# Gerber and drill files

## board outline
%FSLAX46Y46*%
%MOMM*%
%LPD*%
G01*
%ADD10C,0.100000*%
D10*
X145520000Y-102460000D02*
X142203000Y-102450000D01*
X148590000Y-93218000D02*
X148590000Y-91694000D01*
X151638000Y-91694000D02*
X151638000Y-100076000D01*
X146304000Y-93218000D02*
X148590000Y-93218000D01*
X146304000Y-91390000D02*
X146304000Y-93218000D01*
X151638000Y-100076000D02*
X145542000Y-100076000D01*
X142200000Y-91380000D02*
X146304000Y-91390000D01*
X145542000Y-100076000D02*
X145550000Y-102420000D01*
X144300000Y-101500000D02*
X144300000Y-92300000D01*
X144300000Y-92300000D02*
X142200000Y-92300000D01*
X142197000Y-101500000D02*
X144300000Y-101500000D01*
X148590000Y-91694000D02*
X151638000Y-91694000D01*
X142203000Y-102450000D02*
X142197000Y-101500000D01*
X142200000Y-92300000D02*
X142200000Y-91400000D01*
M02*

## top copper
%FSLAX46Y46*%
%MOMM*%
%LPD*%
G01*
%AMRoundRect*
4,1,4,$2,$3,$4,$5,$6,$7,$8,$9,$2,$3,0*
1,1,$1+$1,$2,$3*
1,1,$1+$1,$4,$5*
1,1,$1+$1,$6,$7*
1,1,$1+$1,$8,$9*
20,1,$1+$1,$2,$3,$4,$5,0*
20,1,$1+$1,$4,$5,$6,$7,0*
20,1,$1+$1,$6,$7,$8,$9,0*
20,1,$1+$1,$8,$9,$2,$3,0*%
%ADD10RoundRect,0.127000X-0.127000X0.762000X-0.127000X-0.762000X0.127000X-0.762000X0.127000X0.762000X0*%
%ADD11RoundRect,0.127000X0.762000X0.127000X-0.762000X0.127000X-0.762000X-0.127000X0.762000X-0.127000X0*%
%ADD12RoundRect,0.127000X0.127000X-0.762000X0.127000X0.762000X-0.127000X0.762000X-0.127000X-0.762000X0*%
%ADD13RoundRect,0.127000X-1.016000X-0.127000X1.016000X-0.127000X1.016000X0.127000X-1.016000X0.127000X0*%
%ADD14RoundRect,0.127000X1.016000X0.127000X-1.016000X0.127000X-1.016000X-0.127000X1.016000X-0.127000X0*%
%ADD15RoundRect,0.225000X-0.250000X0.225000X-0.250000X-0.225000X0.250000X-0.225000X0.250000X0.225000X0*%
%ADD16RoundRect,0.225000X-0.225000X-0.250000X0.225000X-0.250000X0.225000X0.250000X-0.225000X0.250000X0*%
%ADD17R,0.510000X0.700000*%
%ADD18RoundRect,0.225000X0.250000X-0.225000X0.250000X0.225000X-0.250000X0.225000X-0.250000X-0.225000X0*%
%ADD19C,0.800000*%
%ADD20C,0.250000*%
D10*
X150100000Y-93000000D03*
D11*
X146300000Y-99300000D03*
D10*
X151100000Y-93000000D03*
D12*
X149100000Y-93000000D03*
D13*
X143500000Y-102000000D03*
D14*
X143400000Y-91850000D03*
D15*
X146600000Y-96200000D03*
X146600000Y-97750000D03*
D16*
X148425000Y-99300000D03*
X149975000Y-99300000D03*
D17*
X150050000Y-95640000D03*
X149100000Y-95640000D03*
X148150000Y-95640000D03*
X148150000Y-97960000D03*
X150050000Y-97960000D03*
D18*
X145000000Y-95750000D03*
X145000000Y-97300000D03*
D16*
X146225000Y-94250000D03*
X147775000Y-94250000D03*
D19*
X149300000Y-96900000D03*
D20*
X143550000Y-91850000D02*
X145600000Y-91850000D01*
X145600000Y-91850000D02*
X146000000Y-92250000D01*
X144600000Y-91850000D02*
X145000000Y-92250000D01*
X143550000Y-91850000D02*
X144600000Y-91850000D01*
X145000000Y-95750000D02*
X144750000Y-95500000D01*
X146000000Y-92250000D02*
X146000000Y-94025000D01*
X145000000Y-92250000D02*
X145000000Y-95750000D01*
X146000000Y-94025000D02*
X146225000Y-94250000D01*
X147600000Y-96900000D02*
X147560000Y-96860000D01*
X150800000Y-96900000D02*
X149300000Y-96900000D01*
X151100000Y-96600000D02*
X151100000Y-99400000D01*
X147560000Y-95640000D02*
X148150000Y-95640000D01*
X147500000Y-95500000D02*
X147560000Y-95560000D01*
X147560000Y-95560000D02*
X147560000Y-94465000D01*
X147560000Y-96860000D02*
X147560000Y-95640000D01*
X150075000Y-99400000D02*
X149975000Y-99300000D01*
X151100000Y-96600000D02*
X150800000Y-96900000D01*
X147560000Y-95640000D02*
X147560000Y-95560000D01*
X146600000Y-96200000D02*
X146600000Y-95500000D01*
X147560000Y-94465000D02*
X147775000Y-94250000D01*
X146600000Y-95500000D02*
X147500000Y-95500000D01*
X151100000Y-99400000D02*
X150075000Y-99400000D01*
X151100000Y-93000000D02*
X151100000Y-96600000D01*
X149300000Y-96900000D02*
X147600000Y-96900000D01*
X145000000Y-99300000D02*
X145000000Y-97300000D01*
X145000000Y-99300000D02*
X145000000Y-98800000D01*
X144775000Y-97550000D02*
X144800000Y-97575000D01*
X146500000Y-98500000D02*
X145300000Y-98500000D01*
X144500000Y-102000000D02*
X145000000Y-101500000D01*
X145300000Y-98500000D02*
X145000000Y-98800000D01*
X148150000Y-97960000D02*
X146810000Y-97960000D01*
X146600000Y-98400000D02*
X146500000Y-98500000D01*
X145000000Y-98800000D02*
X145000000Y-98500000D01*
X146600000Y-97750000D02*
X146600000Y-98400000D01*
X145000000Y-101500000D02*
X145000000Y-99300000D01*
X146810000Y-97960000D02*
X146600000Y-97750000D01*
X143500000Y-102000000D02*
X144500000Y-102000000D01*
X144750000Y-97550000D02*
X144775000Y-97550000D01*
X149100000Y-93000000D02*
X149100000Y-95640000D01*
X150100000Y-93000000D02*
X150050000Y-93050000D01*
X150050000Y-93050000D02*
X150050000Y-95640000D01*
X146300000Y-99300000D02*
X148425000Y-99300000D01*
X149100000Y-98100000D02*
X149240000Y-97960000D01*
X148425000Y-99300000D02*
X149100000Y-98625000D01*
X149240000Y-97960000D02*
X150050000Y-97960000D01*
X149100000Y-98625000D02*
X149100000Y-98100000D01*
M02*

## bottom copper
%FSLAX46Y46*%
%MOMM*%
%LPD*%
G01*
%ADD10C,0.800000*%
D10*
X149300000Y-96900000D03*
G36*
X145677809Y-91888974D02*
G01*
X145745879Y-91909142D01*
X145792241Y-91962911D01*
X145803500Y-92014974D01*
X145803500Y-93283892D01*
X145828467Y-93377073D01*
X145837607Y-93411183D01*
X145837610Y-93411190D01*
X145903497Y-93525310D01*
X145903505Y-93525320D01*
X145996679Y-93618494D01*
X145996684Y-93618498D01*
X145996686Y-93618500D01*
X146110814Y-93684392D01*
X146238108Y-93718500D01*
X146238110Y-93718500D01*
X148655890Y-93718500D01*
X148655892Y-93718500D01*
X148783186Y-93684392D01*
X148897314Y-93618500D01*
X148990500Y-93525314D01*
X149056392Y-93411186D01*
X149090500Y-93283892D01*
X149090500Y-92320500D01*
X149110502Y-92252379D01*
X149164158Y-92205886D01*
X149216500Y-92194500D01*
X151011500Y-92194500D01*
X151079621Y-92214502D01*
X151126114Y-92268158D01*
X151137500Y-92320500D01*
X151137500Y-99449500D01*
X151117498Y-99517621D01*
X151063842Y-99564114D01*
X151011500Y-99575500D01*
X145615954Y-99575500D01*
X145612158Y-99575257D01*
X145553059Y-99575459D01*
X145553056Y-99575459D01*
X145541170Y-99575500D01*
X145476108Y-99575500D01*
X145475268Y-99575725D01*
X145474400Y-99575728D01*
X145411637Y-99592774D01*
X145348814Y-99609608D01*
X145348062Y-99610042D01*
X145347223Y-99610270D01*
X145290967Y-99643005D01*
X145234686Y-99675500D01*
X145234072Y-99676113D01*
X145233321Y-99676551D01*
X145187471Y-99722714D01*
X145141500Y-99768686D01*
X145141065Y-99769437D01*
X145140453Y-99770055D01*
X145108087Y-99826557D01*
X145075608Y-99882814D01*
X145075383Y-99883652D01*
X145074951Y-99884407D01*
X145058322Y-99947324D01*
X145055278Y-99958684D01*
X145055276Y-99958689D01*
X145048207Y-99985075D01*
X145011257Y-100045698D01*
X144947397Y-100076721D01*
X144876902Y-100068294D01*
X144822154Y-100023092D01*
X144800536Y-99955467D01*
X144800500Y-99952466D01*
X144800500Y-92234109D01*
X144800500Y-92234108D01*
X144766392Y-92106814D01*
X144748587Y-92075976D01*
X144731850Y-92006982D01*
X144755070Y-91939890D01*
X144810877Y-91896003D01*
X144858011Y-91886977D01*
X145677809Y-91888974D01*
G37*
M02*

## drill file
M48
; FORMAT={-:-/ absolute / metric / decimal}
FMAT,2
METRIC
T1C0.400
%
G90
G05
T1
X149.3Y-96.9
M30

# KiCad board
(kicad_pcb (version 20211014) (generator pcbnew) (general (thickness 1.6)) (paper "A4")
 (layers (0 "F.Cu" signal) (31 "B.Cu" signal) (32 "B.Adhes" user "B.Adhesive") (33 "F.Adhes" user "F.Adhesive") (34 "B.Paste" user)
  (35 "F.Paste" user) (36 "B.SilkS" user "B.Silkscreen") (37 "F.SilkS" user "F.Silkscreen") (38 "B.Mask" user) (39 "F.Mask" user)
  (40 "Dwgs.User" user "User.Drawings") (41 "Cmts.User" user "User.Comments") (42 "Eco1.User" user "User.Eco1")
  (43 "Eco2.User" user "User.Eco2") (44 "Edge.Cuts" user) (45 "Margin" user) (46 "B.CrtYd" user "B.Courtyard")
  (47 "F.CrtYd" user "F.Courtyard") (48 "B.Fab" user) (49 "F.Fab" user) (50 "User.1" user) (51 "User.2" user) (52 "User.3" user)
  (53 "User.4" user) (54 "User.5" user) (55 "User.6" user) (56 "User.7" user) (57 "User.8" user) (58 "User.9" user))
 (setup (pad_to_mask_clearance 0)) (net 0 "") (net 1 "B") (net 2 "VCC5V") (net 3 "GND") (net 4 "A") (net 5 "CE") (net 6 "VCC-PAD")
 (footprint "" (layer "F.Cu") (at 150.1 93 90)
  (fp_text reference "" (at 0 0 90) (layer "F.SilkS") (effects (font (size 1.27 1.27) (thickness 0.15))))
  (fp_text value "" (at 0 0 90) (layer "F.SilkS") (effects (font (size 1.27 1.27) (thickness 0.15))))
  (pad "B" smd roundrect (at 0 0 270) (size 1.778 0.508) (layers "F.Cu" "F.Paste" "F.Mask") (roundrect_rratio 0.25) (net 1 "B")))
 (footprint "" (layer "F.Cu") (at 146.3 99.3 -90)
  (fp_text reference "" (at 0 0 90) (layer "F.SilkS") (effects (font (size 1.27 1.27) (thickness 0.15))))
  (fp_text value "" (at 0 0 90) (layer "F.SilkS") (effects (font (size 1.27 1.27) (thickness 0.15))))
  (pad "B" smd roundrect (at 0 0 180) (size 1.778 0.508) (layers "F.Cu" "F.Paste" "F.Mask") (roundrect_rratio 0.25) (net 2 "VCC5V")))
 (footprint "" (layer "F.Cu") (at 151.1 93 90)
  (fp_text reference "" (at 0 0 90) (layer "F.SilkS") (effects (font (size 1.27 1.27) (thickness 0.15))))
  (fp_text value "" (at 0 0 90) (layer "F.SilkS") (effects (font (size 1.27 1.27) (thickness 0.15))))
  (pad "1" smd roundrect (at 0 0 270) (size 1.778 0.508) (layers "F.Cu" "F.Paste" "F.Mask") (roundrect_rratio 0.25) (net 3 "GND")))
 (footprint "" (layer "F.Cu") (at 149.1 93 -90)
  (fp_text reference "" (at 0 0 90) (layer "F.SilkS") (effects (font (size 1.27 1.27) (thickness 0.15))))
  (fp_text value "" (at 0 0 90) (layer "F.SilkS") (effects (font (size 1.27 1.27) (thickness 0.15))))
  (pad "1" smd roundrect (at 0 0 90) (size 1.778 0.508) (layers "F.Cu" "F.Paste" "F.Mask") (roundrect_rratio 0.25) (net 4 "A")))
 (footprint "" (layer "F.Cu") (at 143.5 102)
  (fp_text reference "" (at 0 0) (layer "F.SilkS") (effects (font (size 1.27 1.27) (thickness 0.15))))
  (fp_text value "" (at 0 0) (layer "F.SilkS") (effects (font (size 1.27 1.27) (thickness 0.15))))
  (pad "4" smd roundrect (at 0 0) (size 2.286 0.508) (layers "F.Cu" "F.Paste" "F.Mask") (roundrect_rratio 0.25) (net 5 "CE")))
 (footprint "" (layer "F.Cu") (at 143.4 91.85 180)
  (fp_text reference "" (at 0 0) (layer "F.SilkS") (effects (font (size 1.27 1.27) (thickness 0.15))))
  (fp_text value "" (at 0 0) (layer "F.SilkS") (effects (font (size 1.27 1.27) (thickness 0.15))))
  (pad "1" smd roundrect (at 0 0 180) (size 2.286 0.508) (layers "F.Cu" "F.Paste" "F.Mask") (roundrect_rratio 0.25) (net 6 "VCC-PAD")))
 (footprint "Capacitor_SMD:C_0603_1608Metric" (layer "F.Cu") (at 146.6 96.975 -90)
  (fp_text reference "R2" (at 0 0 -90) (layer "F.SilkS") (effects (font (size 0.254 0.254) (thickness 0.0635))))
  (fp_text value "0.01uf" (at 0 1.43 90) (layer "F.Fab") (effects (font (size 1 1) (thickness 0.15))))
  (pad "5" smd roundrect (at -0.775 0 270) (size 0.9 0.95) (layers "F.Cu" "F.Paste" "F.Mask") (roundrect_rratio 0.25) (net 3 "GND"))
  (pad "6" smd roundrect (at 0.775 0 270) (size 0.9 0.95) (layers "F.Cu" "F.Paste" "F.Mask") (roundrect_rratio 0.25) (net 5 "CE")))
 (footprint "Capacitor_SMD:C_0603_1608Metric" (layer "F.Cu") (at 149.2 99.3)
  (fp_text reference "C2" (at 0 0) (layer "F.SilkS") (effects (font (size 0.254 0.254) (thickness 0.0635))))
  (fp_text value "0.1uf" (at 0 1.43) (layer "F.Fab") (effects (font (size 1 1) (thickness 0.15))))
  (pad "5" smd roundrect (at -0.775 0) (size 0.9 0.95) (layers "F.Cu" "F.Paste" "F.Mask") (roundrect_rratio 0.25) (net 2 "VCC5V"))
  (pad "6" smd roundrect (at 0.775 0) (size 0.9 0.95) (layers "F.Cu" "F.Paste" "F.Mask") (roundrect_rratio 0.25) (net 3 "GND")))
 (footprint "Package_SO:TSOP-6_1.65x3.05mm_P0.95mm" (layer "F.Cu") (at 149.1 96.8 -90)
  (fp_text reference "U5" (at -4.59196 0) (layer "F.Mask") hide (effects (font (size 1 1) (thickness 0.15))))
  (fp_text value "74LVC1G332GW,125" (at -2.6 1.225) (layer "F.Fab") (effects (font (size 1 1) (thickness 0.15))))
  (pad "1" smd rect (at -1.16 -0.95 270) (size 0.7 0.51) (layers "F.Cu" "F.Paste" "F.Mask") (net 1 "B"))
  (pad "2" smd rect (at -1.16 0 270) (size 0.7 0.51) (layers "F.Cu" "F.Paste" "F.Mask") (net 4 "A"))
  (pad "3" smd rect (at -1.16 0.95 270) (size 0.7 0.51) (layers "F.Cu" "F.Paste" "F.Mask") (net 3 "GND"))
  (pad "4" smd rect (at 1.16 0.95 270) (size 0.7 0.51) (layers "F.Cu" "F.Paste" "F.Mask") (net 5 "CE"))
  (pad "6" smd rect (at 1.16 -0.95 270) (size 0.7 0.51) (layers "F.Cu" "F.Paste" "F.Mask") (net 2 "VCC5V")))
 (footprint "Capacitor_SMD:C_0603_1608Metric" (layer "F.Cu") (at 145 96.525 90)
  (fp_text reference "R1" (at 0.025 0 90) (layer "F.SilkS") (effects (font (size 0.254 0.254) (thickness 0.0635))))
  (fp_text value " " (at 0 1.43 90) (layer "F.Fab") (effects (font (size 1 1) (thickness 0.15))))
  (pad "2" smd roundrect (at 0.775 0 90) (size 0.9 0.95) (layers "F.Cu" "F.Paste" "F.Mask") (roundrect_rratio 0.25) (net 6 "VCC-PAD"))
  (pad "3" smd roundrect (at -0.775 0 90) (size 0.9 0.95) (layers "F.Cu" "F.Paste" "F.Mask") (roundrect_rratio 0.25) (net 5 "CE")))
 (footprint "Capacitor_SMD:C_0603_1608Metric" (layer "F.Cu") (at 147 94.25)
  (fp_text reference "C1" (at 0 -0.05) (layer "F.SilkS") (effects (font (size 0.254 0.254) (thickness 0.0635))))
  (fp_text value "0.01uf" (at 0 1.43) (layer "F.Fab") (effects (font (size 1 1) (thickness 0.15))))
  (pad "5" smd roundrect (at -0.775 0) (size 0.9 0.95) (layers "F.Cu" "F.Paste" "F.Mask") (roundrect_rratio 0.25) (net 6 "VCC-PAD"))
  (pad "6" smd roundrect (at 0.775 0) (size 0.9 0.95) (layers "F.Cu" "F.Paste" "F.Mask") (roundrect_rratio 0.25) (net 3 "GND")))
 (gr_line (start 145.52 102.46) (end 142.203 102.45) (layer "Edge.Cuts") (width 0.1))
 (gr_line (start 148.59 93.218) (end 148.59 91.694) (layer "Edge.Cuts") (width 0.1))
 (gr_line (start 151.638 91.694) (end 151.638 100.076) (layer "Edge.Cuts") (width 0.1))
 (gr_line (start 146.304 93.218) (end 148.59 93.218) (layer "Edge.Cuts") (width 0.1))
 (gr_line (start 146.304 91.39) (end 146.304 93.218) (layer "Edge.Cuts") (width 0.1))
 (gr_line (start 151.638 100.076) (end 145.542 100.076) (layer "Edge.Cuts") (width 0.1))
 (gr_line (start 142.2 91.38) (end 146.304 91.39) (layer "Edge.Cuts") (width 0.1))
 (gr_line (start 145.542 100.076) (end 145.55 102.42) (layer "Edge.Cuts") (width 0.1))
 (gr_line (start 144.3 101.5) (end 144.3 92.3) (layer "Edge.Cuts") (width 0.1))
 (gr_line (start 144.3 92.3) (end 142.2 92.3) (layer "Edge.Cuts") (width 0.1))
 (gr_line (start 142.197 101.5) (end 144.3 101.5) (layer "Edge.Cuts") (width 0.1))
 (gr_line (start 148.59 91.694) (end 151.638 91.694) (layer "Edge.Cuts") (width 0.1))
 (gr_line (start 142.203 102.45) (end 142.197 101.5) (layer "Edge.Cuts") (width 0.1))
 (gr_line (start 142.2 92.3) (end 142.2 91.4) (layer "Edge.Cuts") (width 0.1))
 (segment (start 143.55 91.85) (end 145.6 91.85) (width 0.25) (layer "F.Cu") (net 6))
 (segment (start 145.6 91.85) (end 146 92.25) (width 0.25) (layer "F.Cu") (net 6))
 (segment (start 144.6 91.85) (end 145 92.25) (width 0.25) (layer "F.Cu") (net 6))
 (segment (start 143.55 91.85) (end 144.6 91.85) (width 0.25) (layer "F.Cu") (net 6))
 (segment (start 145 95.75) (end 144.75 95.5) (width 0.25) (layer "F.Cu") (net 6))
 (segment (start 146 92.25) (end 146 94.025) (width 0.25) (layer "F.Cu") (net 6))
 (segment (start 145 92.25) (end 145 95.75) (width 0.25) (layer "F.Cu") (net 6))
 (segment (start 146 94.025) (end 146.225 94.25) (width 0.25) (layer "F.Cu") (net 6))
 (segment (start 147.6 96.9) (end 147.56 96.86) (width 0.25) (layer "F.Cu") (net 3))
 (segment (start 150.8 96.9) (end 149.3 96.9) (width 0.25) (layer "F.Cu") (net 3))
 (segment (start 151.1 96.6) (end 151.1 99.4) (width 0.25) (layer "F.Cu") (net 3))
 (segment (start 147.56 95.64) (end 148.15 95.64) (width 0.25) (layer "F.Cu") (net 3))
 (segment (start 147.5 95.5) (end 147.56 95.56) (width 0.25) (layer "F.Cu") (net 3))
 (segment (start 147.56 95.56) (end 147.56 94.465) (width 0.25) (layer "F.Cu") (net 3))
 (segment (start 147.56 96.86) (end 147.56 95.64) (width 0.25) (layer "F.Cu") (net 3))
 (segment (start 150.075 99.4) (end 149.975 99.3) (width 0.25) (layer "F.Cu") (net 3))
 (segment (start 151.1 96.6) (end 150.8 96.9) (width 0.25) (layer "F.Cu") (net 3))
 (segment (start 147.56 95.64) (end 147.56 95.56) (width 0.25) (layer "F.Cu") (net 3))
 (segment (start 146.6 96.2) (end 146.6 95.5) (width 0.25) (layer "F.Cu") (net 3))
 (segment (start 147.56 94.465) (end 147.775 94.25) (width 0.25) (layer "F.Cu") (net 3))
 (segment (start 146.6 95.5) (end 147.5 95.5) (width 0.25) (layer "F.Cu") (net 3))
 (segment (start 151.1 99.4) (end 150.075 99.4) (width 0.25) (layer "F.Cu") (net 3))
 (segment (start 151.1 93) (end 151.1 96.6) (width 0.25) (layer "F.Cu") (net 3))
 (segment (start 149.3 96.9) (end 147.6 96.9) (width 0.25) (layer "F.Cu") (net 3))
 (via (at 149.3 96.9) (size 0.8) (drill 0.4) (layers "F.Cu" "B.Cu") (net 3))
 (segment (start 145 99.3) (end 145 97.3) (width 0.25) (layer "F.Cu") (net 5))
 (segment (start 145 99.3) (end 145 98.8) (width 0.25) (layer "F.Cu") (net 5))
 (segment (start 144.775 97.55) (end 144.8 97.575) (width 0.25) (layer "F.Cu") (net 5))
 (segment (start 146.5 98.5) (end 145.3 98.5) (width 0.25) (layer "F.Cu") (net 5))
 (segment (start 144.5 102) (end 145 101.5) (width 0.25) (layer "F.Cu") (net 5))
 (segment (start 145.3 98.5) (end 145 98.8) (width 0.25) (layer "F.Cu") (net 5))
 (segment (start 148.15 97.96) (end 146.81 97.96) (width 0.25) (layer "F.Cu") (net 5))
 (segment (start 146.6 98.4) (end 146.5 98.5) (width 0.25) (layer "F.Cu") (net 5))
 (segment (start 145 98.8) (end 145 98.5) (width 0.25) (layer "F.Cu") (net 5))
 (segment (start 146.6 97.75) (end 146.6 98.4) (width 0.25) (layer "F.Cu") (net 5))
 (segment (start 145 101.5) (end 145 99.3) (width 0.25) (layer "F.Cu") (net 5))
 (segment (start 146.81 97.96) (end 146.6 97.75) (width 0.25) (layer "F.Cu") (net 5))
 (segment (start 143.5 102) (end 144.5 102) (width 0.25) (layer "F.Cu") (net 5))
 (segment (start 144.75 97.55) (end 144.775 97.55) (width 0.25) (layer "F.Cu") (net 5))
 (segment (start 149.1 93) (end 149.1 95.64) (width 0.25) (layer "F.Cu") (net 4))
 (segment (start 150.1 93) (end 150.05 93.05) (width 0.25) (layer "F.Cu") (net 1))
 (segment (start 150.05 93.05) (end 150.05 95.64) (width 0.25) (layer "F.Cu") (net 1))
 (segment (start 146.3 99.3) (end 148.425 99.3) (width 0.25) (layer "F.Cu") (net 2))
 (segment (start 149.1 98.1) (end 149.24 97.96) (width 0.25) (layer "F.Cu") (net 2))
 (segment (start 148.425 99.3) (end 149.1 98.625) (width 0.25) (layer "F.Cu") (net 2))
 (segment (start 149.24 97.96) (end 150.05 97.96) (width 0.25) (layer "F.Cu") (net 2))
 (segment (start 149.1 98.625) (end 149.1 98.1) (width 0.25) (layer "F.Cu") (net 2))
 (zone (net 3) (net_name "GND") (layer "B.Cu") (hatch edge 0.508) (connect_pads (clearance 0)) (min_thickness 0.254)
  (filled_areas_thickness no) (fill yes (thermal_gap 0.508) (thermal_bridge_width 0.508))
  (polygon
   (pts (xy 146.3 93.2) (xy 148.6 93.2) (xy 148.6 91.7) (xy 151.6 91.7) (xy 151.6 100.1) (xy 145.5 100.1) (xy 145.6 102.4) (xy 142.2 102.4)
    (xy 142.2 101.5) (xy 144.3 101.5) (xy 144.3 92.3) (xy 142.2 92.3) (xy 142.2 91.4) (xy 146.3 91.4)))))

